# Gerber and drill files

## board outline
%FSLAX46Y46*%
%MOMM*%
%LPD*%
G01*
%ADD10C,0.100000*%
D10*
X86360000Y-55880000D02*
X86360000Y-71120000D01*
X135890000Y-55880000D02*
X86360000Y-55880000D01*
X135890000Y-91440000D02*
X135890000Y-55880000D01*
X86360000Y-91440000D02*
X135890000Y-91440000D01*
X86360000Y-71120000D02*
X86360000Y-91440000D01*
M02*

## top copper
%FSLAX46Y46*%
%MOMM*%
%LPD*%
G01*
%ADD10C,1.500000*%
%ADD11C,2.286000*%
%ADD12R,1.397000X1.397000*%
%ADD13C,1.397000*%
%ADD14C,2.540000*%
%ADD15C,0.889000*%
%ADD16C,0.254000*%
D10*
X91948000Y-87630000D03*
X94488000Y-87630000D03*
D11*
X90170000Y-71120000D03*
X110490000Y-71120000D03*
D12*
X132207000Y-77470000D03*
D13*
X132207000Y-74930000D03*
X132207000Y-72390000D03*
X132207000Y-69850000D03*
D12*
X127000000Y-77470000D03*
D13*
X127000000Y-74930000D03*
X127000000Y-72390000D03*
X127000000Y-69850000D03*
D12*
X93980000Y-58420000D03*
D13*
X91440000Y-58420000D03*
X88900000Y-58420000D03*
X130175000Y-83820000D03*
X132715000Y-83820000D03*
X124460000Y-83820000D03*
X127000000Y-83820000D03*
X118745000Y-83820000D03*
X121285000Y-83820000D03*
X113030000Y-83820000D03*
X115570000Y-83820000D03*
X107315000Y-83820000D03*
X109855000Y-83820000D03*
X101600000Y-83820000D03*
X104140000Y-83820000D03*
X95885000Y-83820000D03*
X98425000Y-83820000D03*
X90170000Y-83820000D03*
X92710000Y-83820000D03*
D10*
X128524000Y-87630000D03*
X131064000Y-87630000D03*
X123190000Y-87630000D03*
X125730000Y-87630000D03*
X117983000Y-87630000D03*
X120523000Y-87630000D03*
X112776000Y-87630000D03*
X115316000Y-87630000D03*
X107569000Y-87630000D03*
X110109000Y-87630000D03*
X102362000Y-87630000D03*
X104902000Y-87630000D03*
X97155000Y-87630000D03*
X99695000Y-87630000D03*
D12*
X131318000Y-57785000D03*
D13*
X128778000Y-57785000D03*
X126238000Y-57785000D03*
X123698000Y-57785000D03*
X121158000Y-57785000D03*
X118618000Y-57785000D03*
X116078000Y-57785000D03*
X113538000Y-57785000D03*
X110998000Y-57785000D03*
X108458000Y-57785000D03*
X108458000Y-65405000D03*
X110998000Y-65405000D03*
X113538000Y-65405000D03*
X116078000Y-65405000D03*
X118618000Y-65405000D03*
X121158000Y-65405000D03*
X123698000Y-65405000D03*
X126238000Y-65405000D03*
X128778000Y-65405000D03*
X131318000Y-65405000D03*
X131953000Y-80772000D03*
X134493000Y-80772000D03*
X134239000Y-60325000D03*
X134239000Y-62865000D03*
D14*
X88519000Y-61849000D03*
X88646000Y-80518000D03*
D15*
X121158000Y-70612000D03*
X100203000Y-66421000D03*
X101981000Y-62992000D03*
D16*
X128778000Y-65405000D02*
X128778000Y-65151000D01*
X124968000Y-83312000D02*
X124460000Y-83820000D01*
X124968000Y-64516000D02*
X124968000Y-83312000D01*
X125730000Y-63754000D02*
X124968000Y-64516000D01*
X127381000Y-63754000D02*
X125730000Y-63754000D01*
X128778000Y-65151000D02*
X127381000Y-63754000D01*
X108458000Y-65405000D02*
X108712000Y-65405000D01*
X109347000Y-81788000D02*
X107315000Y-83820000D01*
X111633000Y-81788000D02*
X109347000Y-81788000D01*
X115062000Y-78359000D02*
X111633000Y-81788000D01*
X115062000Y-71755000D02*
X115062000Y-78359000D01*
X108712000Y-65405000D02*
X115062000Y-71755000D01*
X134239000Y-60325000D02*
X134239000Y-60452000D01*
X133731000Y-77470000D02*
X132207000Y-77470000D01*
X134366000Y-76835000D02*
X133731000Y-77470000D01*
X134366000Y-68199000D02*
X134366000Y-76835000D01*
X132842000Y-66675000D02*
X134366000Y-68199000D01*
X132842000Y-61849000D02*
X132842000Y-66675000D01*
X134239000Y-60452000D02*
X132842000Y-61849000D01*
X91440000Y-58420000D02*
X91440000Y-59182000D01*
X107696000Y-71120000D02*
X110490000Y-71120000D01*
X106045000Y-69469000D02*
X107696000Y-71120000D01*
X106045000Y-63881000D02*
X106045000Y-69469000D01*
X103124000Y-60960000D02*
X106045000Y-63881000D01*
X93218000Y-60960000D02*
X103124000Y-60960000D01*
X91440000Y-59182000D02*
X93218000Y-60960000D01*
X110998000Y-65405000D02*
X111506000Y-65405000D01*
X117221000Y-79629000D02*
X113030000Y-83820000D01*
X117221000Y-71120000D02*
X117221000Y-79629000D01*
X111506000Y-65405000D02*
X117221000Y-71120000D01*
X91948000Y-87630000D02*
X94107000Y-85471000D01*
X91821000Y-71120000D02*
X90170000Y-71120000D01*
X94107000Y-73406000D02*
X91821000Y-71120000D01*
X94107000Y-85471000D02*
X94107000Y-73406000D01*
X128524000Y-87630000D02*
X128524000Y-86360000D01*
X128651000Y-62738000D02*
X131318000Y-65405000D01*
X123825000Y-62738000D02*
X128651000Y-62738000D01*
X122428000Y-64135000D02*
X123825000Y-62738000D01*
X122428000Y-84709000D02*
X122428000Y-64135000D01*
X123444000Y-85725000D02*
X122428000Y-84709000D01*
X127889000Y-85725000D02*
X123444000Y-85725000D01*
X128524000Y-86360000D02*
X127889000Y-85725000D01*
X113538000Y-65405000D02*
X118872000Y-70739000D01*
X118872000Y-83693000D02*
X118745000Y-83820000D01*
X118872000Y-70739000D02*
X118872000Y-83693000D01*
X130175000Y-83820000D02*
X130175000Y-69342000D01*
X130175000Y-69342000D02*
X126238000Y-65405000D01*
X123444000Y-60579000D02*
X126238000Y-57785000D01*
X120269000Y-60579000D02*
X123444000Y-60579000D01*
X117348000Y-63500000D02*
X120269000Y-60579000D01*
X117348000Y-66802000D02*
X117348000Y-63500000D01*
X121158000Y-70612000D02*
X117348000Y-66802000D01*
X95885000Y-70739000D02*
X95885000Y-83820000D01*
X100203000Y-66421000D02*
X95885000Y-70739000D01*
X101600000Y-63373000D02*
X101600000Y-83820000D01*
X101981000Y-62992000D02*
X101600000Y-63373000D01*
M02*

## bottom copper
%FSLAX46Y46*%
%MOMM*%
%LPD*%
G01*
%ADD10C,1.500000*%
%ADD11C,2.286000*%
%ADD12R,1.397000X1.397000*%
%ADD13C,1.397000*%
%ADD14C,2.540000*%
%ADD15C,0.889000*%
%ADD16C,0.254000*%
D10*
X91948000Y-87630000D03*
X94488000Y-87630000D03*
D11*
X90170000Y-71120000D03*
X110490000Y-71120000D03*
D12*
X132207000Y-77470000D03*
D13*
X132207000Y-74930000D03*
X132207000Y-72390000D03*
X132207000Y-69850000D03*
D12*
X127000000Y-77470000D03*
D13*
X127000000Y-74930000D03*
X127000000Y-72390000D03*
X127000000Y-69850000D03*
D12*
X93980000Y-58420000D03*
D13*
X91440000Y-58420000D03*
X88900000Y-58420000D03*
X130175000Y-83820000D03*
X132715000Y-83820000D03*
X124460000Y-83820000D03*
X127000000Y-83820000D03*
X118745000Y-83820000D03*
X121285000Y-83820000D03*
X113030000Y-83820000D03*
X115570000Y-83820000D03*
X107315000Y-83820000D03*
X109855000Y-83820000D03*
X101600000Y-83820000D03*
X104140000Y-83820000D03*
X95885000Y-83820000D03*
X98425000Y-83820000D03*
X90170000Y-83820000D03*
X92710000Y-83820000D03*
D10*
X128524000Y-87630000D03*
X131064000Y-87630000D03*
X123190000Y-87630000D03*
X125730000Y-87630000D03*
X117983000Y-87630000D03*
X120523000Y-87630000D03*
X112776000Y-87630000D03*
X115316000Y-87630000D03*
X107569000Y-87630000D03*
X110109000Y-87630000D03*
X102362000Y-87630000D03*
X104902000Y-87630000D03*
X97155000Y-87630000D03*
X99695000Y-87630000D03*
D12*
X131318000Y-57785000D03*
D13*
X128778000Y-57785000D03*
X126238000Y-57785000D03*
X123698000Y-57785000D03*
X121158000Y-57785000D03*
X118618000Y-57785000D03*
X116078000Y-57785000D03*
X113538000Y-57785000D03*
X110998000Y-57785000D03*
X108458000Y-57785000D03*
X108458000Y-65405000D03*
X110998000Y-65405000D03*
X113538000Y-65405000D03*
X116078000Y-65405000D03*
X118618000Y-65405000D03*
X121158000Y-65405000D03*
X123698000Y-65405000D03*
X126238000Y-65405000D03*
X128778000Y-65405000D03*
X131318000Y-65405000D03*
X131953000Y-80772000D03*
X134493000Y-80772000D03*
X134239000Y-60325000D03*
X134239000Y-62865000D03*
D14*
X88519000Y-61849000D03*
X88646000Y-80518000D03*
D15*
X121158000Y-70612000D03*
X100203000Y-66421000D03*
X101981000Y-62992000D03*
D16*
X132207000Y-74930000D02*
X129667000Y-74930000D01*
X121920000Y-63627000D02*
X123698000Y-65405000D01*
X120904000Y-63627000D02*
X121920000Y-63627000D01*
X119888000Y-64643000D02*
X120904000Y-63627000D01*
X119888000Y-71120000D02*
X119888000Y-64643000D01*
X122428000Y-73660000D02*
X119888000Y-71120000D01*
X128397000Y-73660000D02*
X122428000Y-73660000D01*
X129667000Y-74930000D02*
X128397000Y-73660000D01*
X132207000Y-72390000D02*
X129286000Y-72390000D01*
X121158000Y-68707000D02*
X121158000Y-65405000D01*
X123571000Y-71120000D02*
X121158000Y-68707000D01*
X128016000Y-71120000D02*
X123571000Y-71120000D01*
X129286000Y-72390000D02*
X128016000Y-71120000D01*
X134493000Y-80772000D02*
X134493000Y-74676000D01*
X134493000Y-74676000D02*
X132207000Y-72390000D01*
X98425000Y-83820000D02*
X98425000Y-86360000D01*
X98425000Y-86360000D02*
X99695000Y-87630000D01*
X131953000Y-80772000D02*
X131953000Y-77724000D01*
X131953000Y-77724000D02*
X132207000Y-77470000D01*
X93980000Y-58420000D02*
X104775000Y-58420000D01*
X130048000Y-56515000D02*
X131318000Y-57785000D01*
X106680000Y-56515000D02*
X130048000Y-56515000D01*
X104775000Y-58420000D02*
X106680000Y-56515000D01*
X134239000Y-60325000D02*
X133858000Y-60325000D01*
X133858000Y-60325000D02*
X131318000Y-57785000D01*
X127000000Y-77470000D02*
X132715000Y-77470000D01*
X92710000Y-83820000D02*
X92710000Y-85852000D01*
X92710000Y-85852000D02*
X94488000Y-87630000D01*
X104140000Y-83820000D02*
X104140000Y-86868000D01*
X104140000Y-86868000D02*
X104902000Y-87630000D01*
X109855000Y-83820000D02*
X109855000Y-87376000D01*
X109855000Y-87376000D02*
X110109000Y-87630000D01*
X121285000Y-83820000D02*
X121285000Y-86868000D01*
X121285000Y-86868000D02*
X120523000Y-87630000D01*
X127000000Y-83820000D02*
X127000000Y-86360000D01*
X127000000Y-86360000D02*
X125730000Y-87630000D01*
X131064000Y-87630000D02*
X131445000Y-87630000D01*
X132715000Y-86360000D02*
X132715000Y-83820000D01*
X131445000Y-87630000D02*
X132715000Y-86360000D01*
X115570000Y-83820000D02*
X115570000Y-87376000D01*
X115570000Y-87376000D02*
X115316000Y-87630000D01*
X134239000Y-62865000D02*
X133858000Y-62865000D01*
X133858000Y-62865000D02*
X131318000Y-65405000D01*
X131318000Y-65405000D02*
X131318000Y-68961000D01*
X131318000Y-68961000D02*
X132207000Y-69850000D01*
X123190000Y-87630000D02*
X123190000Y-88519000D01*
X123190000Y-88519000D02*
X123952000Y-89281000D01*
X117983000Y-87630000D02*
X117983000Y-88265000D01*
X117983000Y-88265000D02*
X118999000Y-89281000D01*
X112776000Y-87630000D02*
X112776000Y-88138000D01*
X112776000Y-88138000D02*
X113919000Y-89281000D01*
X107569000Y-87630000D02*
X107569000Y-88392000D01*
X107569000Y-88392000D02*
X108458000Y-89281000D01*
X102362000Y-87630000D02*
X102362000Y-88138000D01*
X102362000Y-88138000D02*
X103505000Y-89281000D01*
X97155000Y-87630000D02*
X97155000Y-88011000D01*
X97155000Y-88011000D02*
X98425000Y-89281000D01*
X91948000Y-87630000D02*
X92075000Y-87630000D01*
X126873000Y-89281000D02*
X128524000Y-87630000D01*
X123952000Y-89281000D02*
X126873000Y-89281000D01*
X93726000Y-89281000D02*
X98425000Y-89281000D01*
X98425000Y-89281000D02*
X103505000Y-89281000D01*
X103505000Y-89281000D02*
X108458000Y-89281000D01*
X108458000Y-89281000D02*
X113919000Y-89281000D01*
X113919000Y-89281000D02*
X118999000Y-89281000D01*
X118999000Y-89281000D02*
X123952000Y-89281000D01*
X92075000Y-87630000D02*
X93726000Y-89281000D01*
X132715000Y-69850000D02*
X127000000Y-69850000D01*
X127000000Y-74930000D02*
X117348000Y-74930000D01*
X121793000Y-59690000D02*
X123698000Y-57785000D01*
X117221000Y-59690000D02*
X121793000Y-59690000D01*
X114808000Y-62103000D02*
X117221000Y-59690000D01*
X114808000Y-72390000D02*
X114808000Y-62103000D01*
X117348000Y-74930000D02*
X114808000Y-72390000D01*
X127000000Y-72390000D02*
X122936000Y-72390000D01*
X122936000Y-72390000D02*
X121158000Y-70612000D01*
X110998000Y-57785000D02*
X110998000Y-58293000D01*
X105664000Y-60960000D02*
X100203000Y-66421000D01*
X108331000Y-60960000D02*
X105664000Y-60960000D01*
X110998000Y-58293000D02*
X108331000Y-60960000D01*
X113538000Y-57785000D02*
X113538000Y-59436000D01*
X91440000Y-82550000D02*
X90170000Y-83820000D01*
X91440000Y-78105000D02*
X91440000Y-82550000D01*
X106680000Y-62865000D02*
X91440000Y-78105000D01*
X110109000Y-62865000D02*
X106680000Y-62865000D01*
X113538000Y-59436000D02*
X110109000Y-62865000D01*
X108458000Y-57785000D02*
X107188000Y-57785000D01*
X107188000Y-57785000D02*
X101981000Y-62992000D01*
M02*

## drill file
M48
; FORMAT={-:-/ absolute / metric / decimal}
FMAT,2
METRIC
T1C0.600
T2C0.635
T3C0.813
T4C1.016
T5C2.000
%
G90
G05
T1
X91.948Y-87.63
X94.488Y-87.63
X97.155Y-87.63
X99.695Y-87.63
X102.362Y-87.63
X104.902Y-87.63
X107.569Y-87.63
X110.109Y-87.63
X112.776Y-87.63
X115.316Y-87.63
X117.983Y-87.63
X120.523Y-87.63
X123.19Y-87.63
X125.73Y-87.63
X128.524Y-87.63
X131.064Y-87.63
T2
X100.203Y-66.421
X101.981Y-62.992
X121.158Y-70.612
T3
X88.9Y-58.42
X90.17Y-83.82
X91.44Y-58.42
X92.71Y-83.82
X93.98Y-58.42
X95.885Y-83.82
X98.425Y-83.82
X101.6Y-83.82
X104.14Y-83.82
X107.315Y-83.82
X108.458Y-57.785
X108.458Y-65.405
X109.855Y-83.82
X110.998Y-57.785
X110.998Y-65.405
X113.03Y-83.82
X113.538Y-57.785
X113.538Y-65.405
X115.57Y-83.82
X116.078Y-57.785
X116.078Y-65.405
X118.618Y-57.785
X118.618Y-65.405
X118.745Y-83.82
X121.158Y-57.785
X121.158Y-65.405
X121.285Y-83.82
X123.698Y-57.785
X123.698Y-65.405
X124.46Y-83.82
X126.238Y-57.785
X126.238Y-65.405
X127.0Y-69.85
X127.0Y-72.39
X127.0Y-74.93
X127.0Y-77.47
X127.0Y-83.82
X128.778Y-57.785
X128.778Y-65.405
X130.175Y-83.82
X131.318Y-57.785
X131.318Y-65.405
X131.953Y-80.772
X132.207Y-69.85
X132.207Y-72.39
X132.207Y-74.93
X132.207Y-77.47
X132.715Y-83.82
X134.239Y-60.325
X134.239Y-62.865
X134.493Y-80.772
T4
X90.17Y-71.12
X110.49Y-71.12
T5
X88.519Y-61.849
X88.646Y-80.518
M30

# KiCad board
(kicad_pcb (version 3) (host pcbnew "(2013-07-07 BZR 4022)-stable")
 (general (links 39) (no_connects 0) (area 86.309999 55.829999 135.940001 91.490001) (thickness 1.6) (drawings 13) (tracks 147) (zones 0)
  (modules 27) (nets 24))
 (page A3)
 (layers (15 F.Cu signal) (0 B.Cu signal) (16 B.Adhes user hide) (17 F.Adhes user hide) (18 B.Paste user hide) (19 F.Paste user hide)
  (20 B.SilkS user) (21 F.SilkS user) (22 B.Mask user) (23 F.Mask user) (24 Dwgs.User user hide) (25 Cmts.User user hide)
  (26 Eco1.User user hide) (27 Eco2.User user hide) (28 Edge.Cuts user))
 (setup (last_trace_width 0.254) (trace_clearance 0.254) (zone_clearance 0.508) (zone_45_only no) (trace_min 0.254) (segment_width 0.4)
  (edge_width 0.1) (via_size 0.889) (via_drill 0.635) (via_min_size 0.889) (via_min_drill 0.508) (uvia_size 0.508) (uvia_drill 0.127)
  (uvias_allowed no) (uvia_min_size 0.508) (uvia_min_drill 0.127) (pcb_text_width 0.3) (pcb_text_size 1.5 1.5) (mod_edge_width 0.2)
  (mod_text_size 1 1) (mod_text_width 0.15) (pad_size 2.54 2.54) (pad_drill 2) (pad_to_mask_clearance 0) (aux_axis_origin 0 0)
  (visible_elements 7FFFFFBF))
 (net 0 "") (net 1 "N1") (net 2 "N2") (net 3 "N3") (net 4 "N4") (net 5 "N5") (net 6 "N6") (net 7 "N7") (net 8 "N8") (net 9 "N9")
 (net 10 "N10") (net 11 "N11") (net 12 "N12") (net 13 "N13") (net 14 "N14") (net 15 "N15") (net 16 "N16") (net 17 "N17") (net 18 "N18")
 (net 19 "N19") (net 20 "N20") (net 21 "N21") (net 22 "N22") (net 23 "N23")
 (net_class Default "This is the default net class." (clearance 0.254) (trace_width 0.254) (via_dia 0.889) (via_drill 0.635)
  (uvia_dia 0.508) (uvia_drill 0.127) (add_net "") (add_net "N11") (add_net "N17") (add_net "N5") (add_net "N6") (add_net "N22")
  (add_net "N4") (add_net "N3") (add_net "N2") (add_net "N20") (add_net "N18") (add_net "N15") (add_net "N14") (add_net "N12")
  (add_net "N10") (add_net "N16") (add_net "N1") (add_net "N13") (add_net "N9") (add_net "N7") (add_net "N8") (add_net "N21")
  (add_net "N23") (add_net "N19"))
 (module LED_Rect (layer F.Cu) (at 91.948 87.63)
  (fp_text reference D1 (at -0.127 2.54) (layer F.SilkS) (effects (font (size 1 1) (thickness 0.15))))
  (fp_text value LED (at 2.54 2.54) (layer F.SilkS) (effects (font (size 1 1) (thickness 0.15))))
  (pad 1 thru_hole circle (at 0 0) (size 1.5 1.5) (drill 0.6) (layers *.Cu *.Mask F.SilkS) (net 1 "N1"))
  (pad 2 thru_hole circle (at 2.54 0) (size 1.5 1.5) (drill 0.6) (layers *.Cu *.Mask F.SilkS) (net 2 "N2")))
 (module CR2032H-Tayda (layer F.Cu) (at 97.79 71.12)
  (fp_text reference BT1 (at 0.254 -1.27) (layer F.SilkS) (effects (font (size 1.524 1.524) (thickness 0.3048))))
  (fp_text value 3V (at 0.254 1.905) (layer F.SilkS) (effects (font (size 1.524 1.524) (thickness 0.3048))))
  (pad 2 thru_hole circle (at -7.62 0) (size 2.286 2.286) (drill 1.016) (layers *.Cu *.Mask F.SilkS) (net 1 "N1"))
  (pad 1 thru_hole circle (at 12.7 0) (size 2.286 2.286) (drill 1.016) (layers *.Cu *.Mask F.SilkS) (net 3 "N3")))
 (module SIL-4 (layer F.Cu) (at 132.207 73.66 90)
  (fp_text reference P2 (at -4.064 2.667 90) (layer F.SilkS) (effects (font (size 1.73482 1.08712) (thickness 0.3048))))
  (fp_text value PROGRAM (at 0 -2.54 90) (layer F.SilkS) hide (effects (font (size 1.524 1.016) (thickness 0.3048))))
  (pad 1 thru_hole rect (at -3.81 0 90) (size 1.397 1.397) (drill 0.8128) (layers *.Cu *.Mask F.SilkS) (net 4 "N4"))
  (pad 2 thru_hole circle (at -1.27 0 90) (size 1.397 1.397) (drill 0.8128) (layers *.Cu *.Mask F.SilkS) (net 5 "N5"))
  (pad 3 thru_hole circle (at 1.27 0 90) (size 1.397 1.397) (drill 0.8128) (layers *.Cu *.Mask F.SilkS) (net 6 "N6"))
  (pad 4 thru_hole circle (at 3.81 0 90) (size 1.397 1.397) (drill 0.8128) (layers *.Cu *.Mask F.SilkS) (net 1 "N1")))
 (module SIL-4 (layer F.Cu) (at 127 73.66 90)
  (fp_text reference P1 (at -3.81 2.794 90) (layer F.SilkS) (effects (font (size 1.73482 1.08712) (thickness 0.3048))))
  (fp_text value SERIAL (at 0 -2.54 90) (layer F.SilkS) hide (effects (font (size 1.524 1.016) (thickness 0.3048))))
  (pad 1 thru_hole rect (at -3.81 0 90) (size 1.397 1.397) (drill 0.8128) (layers *.Cu *.Mask F.SilkS) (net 4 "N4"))
  (pad 2 thru_hole circle (at -1.27 0 90) (size 1.397 1.397) (drill 0.8128) (layers *.Cu *.Mask F.SilkS) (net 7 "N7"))
  (pad 3 thru_hole circle (at 1.27 0 90) (size 1.397 1.397) (drill 0.8128) (layers *.Cu *.Mask F.SilkS) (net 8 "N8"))
  (pad 4 thru_hole circle (at 3.81 0 90) (size 1.397 1.397) (drill 0.8128) (layers *.Cu *.Mask F.SilkS) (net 1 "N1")))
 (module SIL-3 (layer F.Cu) (at 91.44 58.42 180)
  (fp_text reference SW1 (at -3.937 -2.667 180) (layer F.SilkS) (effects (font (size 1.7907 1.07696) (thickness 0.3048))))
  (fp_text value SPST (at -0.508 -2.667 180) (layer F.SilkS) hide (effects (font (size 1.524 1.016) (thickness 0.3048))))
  (pad 1 thru_hole rect (at -2.54 0 180) (size 1.397 1.397) (drill 0.8128) (layers *.Cu *.Mask F.SilkS) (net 4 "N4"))
  (pad 2 thru_hole circle (at 0 0 180) (size 1.397 1.397) (drill 0.8128) (layers *.Cu *.Mask F.SilkS) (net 3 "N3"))
  (pad 3 thru_hole circle (at 2.54 0 180) (size 1.397 1.397) (drill 0.8128) (layers *.Cu *.Mask F.SilkS)))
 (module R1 (layer F.Cu) (at 131.445 83.82) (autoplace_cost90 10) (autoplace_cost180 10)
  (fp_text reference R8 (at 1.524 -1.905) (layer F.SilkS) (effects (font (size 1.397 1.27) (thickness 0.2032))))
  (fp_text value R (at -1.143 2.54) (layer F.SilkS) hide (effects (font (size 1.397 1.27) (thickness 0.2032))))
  (pad 1 thru_hole circle (at -1.27 0) (size 1.397 1.397) (drill 0.8128) (layers *.Cu *.Mask F.SilkS) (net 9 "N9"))
  (pad 2 thru_hole circle (at 1.27 0) (size 1.397 1.397) (drill 0.8128) (layers *.Cu *.Mask F.SilkS) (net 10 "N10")))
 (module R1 (layer F.Cu) (at 125.73 83.82) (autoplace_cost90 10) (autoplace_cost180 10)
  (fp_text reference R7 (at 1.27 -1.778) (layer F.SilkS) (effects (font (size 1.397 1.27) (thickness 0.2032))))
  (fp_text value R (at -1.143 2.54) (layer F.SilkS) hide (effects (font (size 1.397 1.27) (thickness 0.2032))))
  (pad 1 thru_hole circle (at -1.27 0) (size 1.397 1.397) (drill 0.8128) (layers *.Cu *.Mask F.SilkS) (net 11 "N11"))
  (pad 2 thru_hole circle (at 1.27 0) (size 1.397 1.397) (drill 0.8128) (layers *.Cu *.Mask F.SilkS) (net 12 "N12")))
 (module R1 (layer F.Cu) (at 120.015 83.82) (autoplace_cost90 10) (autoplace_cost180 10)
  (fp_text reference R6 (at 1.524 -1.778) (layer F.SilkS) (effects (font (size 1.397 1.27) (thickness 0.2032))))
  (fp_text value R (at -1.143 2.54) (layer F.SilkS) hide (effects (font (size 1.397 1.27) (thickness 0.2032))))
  (pad 1 thru_hole circle (at -1.27 0) (size 1.397 1.397) (drill 0.8128) (layers *.Cu *.Mask F.SilkS) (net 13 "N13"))
  (pad 2 thru_hole circle (at 1.27 0) (size 1.397 1.397) (drill 0.8128) (layers *.Cu *.Mask F.SilkS) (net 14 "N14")))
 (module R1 (layer F.Cu) (at 114.3 83.82) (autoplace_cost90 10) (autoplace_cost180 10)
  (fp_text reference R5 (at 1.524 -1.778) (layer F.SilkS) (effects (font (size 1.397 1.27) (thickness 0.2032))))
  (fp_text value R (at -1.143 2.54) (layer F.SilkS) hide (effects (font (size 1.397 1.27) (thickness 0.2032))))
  (pad 1 thru_hole circle (at -1.27 0) (size 1.397 1.397) (drill 0.8128) (layers *.Cu *.Mask F.SilkS) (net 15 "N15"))
  (pad 2 thru_hole circle (at 1.27 0) (size 1.397 1.397) (drill 0.8128) (layers *.Cu *.Mask F.SilkS) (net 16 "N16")))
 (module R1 (layer F.Cu) (at 108.585 83.82) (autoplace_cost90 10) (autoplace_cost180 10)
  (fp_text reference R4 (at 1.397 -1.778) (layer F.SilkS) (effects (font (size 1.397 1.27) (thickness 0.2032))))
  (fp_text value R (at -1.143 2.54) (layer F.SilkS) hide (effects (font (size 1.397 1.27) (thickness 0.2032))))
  (pad 1 thru_hole circle (at -1.27 0) (size 1.397 1.397) (drill 0.8128) (layers *.Cu *.Mask F.SilkS) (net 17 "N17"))
  (pad 2 thru_hole circle (at 1.27 0) (size 1.397 1.397) (drill 0.8128) (layers *.Cu *.Mask F.SilkS) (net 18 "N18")))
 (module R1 (layer F.Cu) (at 102.87 83.82) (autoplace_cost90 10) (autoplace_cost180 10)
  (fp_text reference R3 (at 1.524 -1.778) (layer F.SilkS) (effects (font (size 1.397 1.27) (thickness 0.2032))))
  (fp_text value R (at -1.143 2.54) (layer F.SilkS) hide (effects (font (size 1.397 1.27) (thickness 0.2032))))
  (pad 1 thru_hole circle (at -1.27 0) (size 1.397 1.397) (drill 0.8128) (layers *.Cu *.Mask F.SilkS) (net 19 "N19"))
  (pad 2 thru_hole circle (at 1.27 0) (size 1.397 1.397) (drill 0.8128) (layers *.Cu *.Mask F.SilkS) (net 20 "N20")))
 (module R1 (layer F.Cu) (at 97.155 83.82) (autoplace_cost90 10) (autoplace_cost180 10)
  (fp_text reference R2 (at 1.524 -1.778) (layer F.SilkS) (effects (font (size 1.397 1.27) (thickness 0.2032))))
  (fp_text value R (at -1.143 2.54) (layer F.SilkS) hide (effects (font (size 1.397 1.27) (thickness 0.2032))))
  (pad 1 thru_hole circle (at -1.27 0) (size 1.397 1.397) (drill 0.8128) (layers *.Cu *.Mask F.SilkS) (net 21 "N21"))
  (pad 2 thru_hole circle (at 1.27 0) (size 1.397 1.397) (drill 0.8128) (layers *.Cu *.Mask F.SilkS) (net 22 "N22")))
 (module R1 (layer F.Cu) (at 91.44 83.82) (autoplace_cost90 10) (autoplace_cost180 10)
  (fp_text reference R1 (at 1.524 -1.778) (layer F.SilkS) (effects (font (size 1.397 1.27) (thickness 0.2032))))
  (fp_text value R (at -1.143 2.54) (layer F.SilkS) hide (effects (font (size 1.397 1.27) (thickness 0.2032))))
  (pad 1 thru_hole circle (at -1.27 0) (size 1.397 1.397) (drill 0.8128) (layers *.Cu *.Mask F.SilkS) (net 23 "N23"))
  (pad 2 thru_hole circle (at 1.27 0) (size 1.397 1.397) (drill 0.8128) (layers *.Cu *.Mask F.SilkS) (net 2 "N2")))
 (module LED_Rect (layer F.Cu) (at 128.524 87.63)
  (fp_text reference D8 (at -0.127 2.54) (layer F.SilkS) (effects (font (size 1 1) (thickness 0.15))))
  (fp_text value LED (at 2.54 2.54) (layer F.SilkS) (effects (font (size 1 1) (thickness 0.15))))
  (pad 1 thru_hole circle (at 0 0) (size 1.5 1.5) (drill 0.6) (layers *.Cu *.Mask F.SilkS) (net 1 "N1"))
  (pad 2 thru_hole circle (at 2.54 0) (size 1.5 1.5) (drill 0.6) (layers *.Cu *.Mask F.SilkS) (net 10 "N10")))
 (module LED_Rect (layer F.Cu) (at 123.19 87.63)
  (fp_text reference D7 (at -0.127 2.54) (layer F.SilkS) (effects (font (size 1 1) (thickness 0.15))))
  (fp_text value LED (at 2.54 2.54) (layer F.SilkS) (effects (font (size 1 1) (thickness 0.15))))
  (pad 1 thru_hole circle (at 0 0) (size 1.5 1.5) (drill 0.6) (layers *.Cu *.Mask F.SilkS) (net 1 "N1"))
  (pad 2 thru_hole circle (at 2.54 0) (size 1.5 1.5) (drill 0.6) (layers *.Cu *.Mask F.SilkS) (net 12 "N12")))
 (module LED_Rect (layer F.Cu) (at 117.983 87.63)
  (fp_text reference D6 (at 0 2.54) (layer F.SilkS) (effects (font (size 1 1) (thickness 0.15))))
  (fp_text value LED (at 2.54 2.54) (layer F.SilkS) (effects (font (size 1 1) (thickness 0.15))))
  (pad 1 thru_hole circle (at 0 0) (size 1.5 1.5) (drill 0.6) (layers *.Cu *.Mask F.SilkS) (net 1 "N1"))
  (pad 2 thru_hole circle (at 2.54 0) (size 1.5 1.5) (drill 0.6) (layers *.Cu *.Mask F.SilkS) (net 14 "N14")))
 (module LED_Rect (layer F.Cu) (at 112.776 87.63)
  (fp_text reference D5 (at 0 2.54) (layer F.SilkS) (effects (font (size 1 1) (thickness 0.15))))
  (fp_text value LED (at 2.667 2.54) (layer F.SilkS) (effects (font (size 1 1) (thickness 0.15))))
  (pad 1 thru_hole circle (at 0 0) (size 1.5 1.5) (drill 0.6) (layers *.Cu *.Mask F.SilkS) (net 1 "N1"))
  (pad 2 thru_hole circle (at 2.54 0) (size 1.5 1.5) (drill 0.6) (layers *.Cu *.Mask F.SilkS) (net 16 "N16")))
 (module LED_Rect (layer F.Cu) (at 107.569 87.63)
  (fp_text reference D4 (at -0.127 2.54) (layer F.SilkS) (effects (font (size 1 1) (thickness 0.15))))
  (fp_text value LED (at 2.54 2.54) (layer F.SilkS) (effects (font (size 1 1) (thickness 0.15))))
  (pad 1 thru_hole circle (at 0 0) (size 1.5 1.5) (drill 0.6) (layers *.Cu *.Mask F.SilkS) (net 1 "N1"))
  (pad 2 thru_hole circle (at 2.54 0) (size 1.5 1.5) (drill 0.6) (layers *.Cu *.Mask F.SilkS) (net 18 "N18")))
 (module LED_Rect (layer F.Cu) (at 102.362 87.63)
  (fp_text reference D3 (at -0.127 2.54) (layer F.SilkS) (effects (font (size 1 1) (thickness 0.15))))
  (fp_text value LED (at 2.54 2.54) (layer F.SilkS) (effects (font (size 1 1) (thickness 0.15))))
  (pad 1 thru_hole circle (at 0 0) (size 1.5 1.5) (drill 0.6) (layers *.Cu *.Mask F.SilkS) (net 1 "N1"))
  (pad 2 thru_hole circle (at 2.54 0) (size 1.5 1.5) (drill 0.6) (layers *.Cu *.Mask F.SilkS) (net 20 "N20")))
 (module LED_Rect (layer F.Cu) (at 97.155 87.63)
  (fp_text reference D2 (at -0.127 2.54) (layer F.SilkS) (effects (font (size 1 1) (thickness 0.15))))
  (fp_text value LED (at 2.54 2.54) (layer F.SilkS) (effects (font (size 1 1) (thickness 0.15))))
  (pad 1 thru_hole circle (at 0 0) (size 1.5 1.5) (drill 0.6) (layers *.Cu *.Mask F.SilkS) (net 1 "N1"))
  (pad 2 thru_hole circle (at 2.54 0) (size 1.5 1.5) (drill 0.6) (layers *.Cu *.Mask F.SilkS) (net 22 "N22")))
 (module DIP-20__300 (layer F.Cu) (at 119.888 61.595 180)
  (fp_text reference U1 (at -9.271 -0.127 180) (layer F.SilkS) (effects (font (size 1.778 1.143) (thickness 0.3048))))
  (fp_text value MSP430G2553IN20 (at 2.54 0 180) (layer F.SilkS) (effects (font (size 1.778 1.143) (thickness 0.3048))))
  (pad 1 thru_hole rect (at -11.43 3.81 180) (size 1.397 1.397) (drill 0.8128) (layers *.Cu *.Mask F.SilkS) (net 4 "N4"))
  (pad 2 thru_hole circle (at -8.89 3.81 180) (size 1.397 1.397) (drill 0.8128) (layers *.Cu *.Mask F.SilkS))
  (pad 3 thru_hole circle (at -6.35 3.81 180) (size 1.397 1.397) (drill 0.8128) (layers *.Cu *.Mask F.SilkS) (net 8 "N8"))
  (pad 4 thru_hole circle (at -3.81 3.81 180) (size 1.397 1.397) (drill 0.8128) (layers *.Cu *.Mask F.SilkS) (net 7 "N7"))
  (pad 5 thru_hole circle (at -1.27 3.81 180) (size 1.397 1.397) (drill 0.8128) (layers *.Cu *.Mask F.SilkS))
  (pad 6 thru_hole circle (at 1.27 3.81 180) (size 1.397 1.397) (drill 0.8128) (layers *.Cu *.Mask F.SilkS))
  (pad 7 thru_hole circle (at 3.81 3.81 180) (size 1.397 1.397) (drill 0.8128) (layers *.Cu *.Mask F.SilkS))
  (pad 8 thru_hole circle (at 6.35 3.81 180) (size 1.397 1.397) (drill 0.8128) (layers *.Cu *.Mask F.SilkS) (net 23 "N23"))
  (pad 9 thru_hole circle (at 8.89 3.81 180) (size 1.397 1.397) (drill 0.8128) (layers *.Cu *.Mask F.SilkS) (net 21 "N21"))
  (pad 10 thru_hole circle (at 11.43 3.81 180) (size 1.397 1.397) (drill 0.8128) (layers *.Cu *.Mask F.SilkS) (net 19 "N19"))
  (pad 11 thru_hole circle (at 11.43 -3.81 180) (size 1.397 1.397) (drill 0.8128) (layers *.Cu *.Mask F.SilkS) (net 17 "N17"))
  (pad 12 thru_hole circle (at 8.89 -3.81 180) (size 1.397 1.397) (drill 0.8128) (layers *.Cu *.Mask F.SilkS) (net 15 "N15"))
  (pad 13 thru_hole circle (at 6.35 -3.81 180) (size 1.397 1.397) (drill 0.8128) (layers *.Cu *.Mask F.SilkS) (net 13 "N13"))
  (pad 14 thru_hole circle (at 3.81 -3.81 180) (size 1.397 1.397) (drill 0.8128) (layers *.Cu *.Mask F.SilkS))
  (pad 15 thru_hole circle (at 1.27 -3.81 180) (size 1.397 1.397) (drill 0.8128) (layers *.Cu *.Mask F.SilkS))
  (pad 16 thru_hole circle (at -1.27 -3.81 180) (size 1.397 1.397) (drill 0.8128) (layers *.Cu *.Mask F.SilkS) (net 6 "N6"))
  (pad 17 thru_hole circle (at -3.81 -3.81 180) (size 1.397 1.397) (drill 0.8128) (layers *.Cu *.Mask F.SilkS) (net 5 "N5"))
  (pad 18 thru_hole circle (at -6.35 -3.81 180) (size 1.397 1.397) (drill 0.8128) (layers *.Cu *.Mask F.SilkS) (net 9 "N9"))
  (pad 19 thru_hole circle (at -8.89 -3.81 180) (size 1.397 1.397) (drill 0.8128) (layers *.Cu *.Mask F.SilkS) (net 11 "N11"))
  (pad 20 thru_hole circle (at -11.43 -3.81 180) (size 1.397 1.397) (drill 0.8128) (layers *.Cu *.Mask F.SilkS) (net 1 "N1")))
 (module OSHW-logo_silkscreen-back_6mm (layer F.Cu) (at 97.409 65.405)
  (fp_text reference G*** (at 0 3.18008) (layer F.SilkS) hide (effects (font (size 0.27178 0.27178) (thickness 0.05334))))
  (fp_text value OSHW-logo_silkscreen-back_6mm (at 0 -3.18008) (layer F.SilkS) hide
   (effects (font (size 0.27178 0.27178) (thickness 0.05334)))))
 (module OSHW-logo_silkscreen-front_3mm (layer F.Cu) (at 119.38 68.072)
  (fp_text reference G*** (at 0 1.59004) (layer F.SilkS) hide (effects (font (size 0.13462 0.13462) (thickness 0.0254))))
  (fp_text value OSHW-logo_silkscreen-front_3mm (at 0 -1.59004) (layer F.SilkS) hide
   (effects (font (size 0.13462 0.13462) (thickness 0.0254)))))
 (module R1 (layer F.Cu) (at 133.223 80.772) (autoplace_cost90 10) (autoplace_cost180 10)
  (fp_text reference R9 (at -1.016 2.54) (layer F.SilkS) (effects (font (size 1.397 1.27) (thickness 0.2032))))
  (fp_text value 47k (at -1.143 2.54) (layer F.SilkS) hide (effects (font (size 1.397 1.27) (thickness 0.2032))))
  (pad 1 thru_hole circle (at -1.27 0) (size 1.397 1.397) (drill 0.8128) (layers *.Cu *.Mask F.SilkS) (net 4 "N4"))
  (pad 2 thru_hole circle (at 1.27 0) (size 1.397 1.397) (drill 0.8128) (layers *.Cu *.Mask F.SilkS) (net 6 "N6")))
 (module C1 (layer F.Cu) (at 134.239 61.595 270)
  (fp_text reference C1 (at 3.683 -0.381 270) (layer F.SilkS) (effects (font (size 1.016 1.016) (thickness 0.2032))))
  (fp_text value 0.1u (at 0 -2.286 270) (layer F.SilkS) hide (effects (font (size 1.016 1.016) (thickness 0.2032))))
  (pad 1 thru_hole circle (at -1.27 0 270) (size 1.397 1.397) (drill 0.8128) (layers *.Cu *.Mask F.SilkS) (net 4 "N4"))
  (pad 2 thru_hole circle (at 1.27 0 270) (size 1.397 1.397) (drill 0.8128) (layers *.Cu *.Mask F.SilkS) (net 1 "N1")))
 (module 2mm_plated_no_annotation (layer F.Cu) (at 88.519 61.849)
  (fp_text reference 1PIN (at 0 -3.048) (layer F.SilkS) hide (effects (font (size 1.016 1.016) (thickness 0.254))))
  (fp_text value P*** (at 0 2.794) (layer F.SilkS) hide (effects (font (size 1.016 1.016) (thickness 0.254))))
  (pad "" thru_hole circle (at 0 0) (size 2.54 2.54) (drill 2) (layers *.Cu *.Mask F.SilkS)))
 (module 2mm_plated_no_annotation (layer F.Cu) (at 88.646 80.518)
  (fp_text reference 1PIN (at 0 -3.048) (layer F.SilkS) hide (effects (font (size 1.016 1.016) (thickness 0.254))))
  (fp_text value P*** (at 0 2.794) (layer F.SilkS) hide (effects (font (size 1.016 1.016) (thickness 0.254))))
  (pad "" thru_hole circle (at 0 0) (size 2.54 2.54) (drill 2) (layers *.Cu *.Mask F.SilkS)))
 (gr_line (start 86.36 55.88) (end 86.36 71.12) (angle 90) (layer Edge.Cuts) (width 0.1))
 (gr_line (start 135.89 55.88) (end 86.36 55.88) (angle 90) (layer Edge.Cuts) (width 0.1))
 (gr_line (start 135.89 91.44) (end 135.89 55.88) (angle 90) (layer Edge.Cuts) (width 0.1))
 (gr_line (start 86.36 91.44) (end 135.89 91.44) (angle 90) (layer Edge.Cuts) (width 0.1))
 (gr_line (start 86.36 71.12) (end 86.36 91.44) (angle 90) (layer Edge.Cuts) (width 0.1))
 (segment (start 128.778 65.405) (end 128.778 65.151) (width 0.254) (layer F.Cu) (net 11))
 (segment (start 124.968 83.312) (end 124.46 83.82) (width 0.254) (layer F.Cu) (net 11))
 (segment (start 124.968 64.516) (end 124.968 83.312) (width 0.254) (layer F.Cu) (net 11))
 (segment (start 125.73 63.754) (end 124.968 64.516) (width 0.254) (layer F.Cu) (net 11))
 (segment (start 127.381 63.754) (end 125.73 63.754) (width 0.254) (layer F.Cu) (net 11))
 (segment (start 128.778 65.151) (end 127.381 63.754) (width 0.254) (layer F.Cu) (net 11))
 (segment (start 108.458 65.405) (end 108.712 65.405) (width 0.254) (layer F.Cu) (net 17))
 (segment (start 109.347 81.788) (end 107.315 83.82) (width 0.254) (layer F.Cu) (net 17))
 (segment (start 111.633 81.788) (end 109.347 81.788) (width 0.254) (layer F.Cu) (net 17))
 (segment (start 115.062 78.359) (end 111.633 81.788) (width 0.254) (layer F.Cu) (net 17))
 (segment (start 115.062 71.755) (end 115.062 78.359) (width 0.254) (layer F.Cu) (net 17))
 (segment (start 108.712 65.405) (end 115.062 71.755) (width 0.254) (layer F.Cu) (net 17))
 (segment (start 132.207 74.93) (end 129.667 74.93) (width 0.254) (layer B.Cu) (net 5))
 (segment (start 121.92 63.627) (end 123.698 65.405) (width 0.254) (layer B.Cu) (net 5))
 (segment (start 120.904 63.627) (end 121.92 63.627) (width 0.254) (layer B.Cu) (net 5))
 (segment (start 119.888 64.643) (end 120.904 63.627) (width 0.254) (layer B.Cu) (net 5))
 (segment (start 119.888 71.12) (end 119.888 64.643) (width 0.254) (layer B.Cu) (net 5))
 (segment (start 122.428 73.66) (end 119.888 71.12) (width 0.254) (layer B.Cu) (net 5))
 (segment (start 128.397 73.66) (end 122.428 73.66) (width 0.254) (layer B.Cu) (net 5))
 (segment (start 129.667 74.93) (end 128.397 73.66) (width 0.254) (layer B.Cu) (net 5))
 (segment (start 132.207 72.39) (end 129.286 72.39) (width 0.254) (layer B.Cu) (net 6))
 (segment (start 121.158 68.707) (end 121.158 65.405) (width 0.254) (layer B.Cu) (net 6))
 (segment (start 123.571 71.12) (end 121.158 68.707) (width 0.254) (layer B.Cu) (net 6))
 (segment (start 128.016 71.12) (end 123.571 71.12) (width 0.254) (layer B.Cu) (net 6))
 (segment (start 129.286 72.39) (end 128.016 71.12) (width 0.254) (layer B.Cu) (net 6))
 (segment (start 134.493 80.772) (end 134.493 74.676) (width 0.254) (layer B.Cu) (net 6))
 (segment (start 134.493 74.676) (end 132.207 72.39) (width 0.254) (layer B.Cu) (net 6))
 (segment (start 98.425 83.82) (end 98.425 86.36) (width 0.254) (layer B.Cu) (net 22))
 (segment (start 98.425 86.36) (end 99.695 87.63) (width 0.254) (layer B.Cu) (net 22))
 (segment (start 131.953 80.772) (end 131.953 77.724) (width 0.254) (layer B.Cu) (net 4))
 (segment (start 131.953 77.724) (end 132.207 77.47) (width 0.254) (layer B.Cu) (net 4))
 (segment (start 134.239 60.325) (end 134.239 60.452) (width 0.254) (layer F.Cu) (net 4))
 (segment (start 133.731 77.47) (end 132.207 77.47) (width 0.254) (layer F.Cu) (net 4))
 (segment (start 134.366 76.835) (end 133.731 77.47) (width 0.254) (layer F.Cu) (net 4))
 (segment (start 134.366 68.199) (end 134.366 76.835) (width 0.254) (layer F.Cu) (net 4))
 (segment (start 132.842 66.675) (end 134.366 68.199) (width 0.254) (layer F.Cu) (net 4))
 (segment (start 132.842 61.849) (end 132.842 66.675) (width 0.254) (layer F.Cu) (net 4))
 (segment (start 134.239 60.452) (end 132.842 61.849) (width 0.254) (layer F.Cu) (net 4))
 (segment (start 93.98 58.42) (end 104.775 58.42) (width 0.254) (layer B.Cu) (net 4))
 (segment (start 130.048 56.515) (end 131.318 57.785) (width 0.254) (layer B.Cu) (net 4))
 (segment (start 106.68 56.515) (end 130.048 56.515) (width 0.254) (layer B.Cu) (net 4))
 (segment (start 104.775 58.42) (end 106.68 56.515) (width 0.254) (layer B.Cu) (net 4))
 (segment (start 134.239 60.325) (end 133.858 60.325) (width 0.254) (layer B.Cu) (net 4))
 (segment (start 133.858 60.325) (end 131.318 57.785) (width 0.254) (layer B.Cu) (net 4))
 (segment (start 127 77.47) (end 132.715 77.47) (width 0.254) (layer B.Cu) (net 4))
 (segment (start 91.44 58.42) (end 91.44 59.182) (width 0.254) (layer F.Cu) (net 3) (status 400000))
 (segment (start 107.696 71.12) (end 110.49 71.12) (width 0.254) (layer F.Cu) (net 3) (status 800000))
 (segment (start 106.045 69.469) (end 107.696 71.12) (width 0.254) (layer F.Cu) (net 3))
 (segment (start 106.045 63.881) (end 106.045 69.469) (width 0.254) (layer F.Cu) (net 3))
 (segment (start 103.124 60.96) (end 106.045 63.881) (width 0.254) (layer F.Cu) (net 3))
 (segment (start 93.218 60.96) (end 103.124 60.96) (width 0.254) (layer F.Cu) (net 3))
 (segment (start 91.44 59.182) (end 93.218 60.96) (width 0.254) (layer F.Cu) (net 3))
 (segment (start 92.71 83.82) (end 92.71 85.852) (width 0.254) (layer B.Cu) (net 2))
 (segment (start 92.71 85.852) (end 94.488 87.63) (width 0.254) (layer B.Cu) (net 2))
 (segment (start 104.14 83.82) (end 104.14 86.868) (width 0.254) (layer B.Cu) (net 20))
 (segment (start 104.14 86.868) (end 104.902 87.63) (width 0.254) (layer B.Cu) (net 20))
 (segment (start 109.855 83.82) (end 109.855 87.376) (width 0.254) (layer B.Cu) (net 18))
 (segment (start 109.855 87.376) (end 110.109 87.63) (width 0.254) (layer B.Cu) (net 18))
 (segment (start 110.998 65.405) (end 111.506 65.405) (width 0.254) (layer F.Cu) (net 15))
 (segment (start 117.221 79.629) (end 113.03 83.82) (width 0.254) (layer F.Cu) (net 15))
 (segment (start 117.221 71.12) (end 117.221 79.629) (width 0.254) (layer F.Cu) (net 15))
 (segment (start 111.506 65.405) (end 117.221 71.12) (width 0.254) (layer F.Cu) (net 15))
 (segment (start 121.285 83.82) (end 121.285 86.868) (width 0.254) (layer B.Cu) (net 14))
 (segment (start 121.285 86.868) (end 120.523 87.63) (width 0.254) (layer B.Cu) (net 14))
 (segment (start 127 83.82) (end 127 86.36) (width 0.254) (layer B.Cu) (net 12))
 (segment (start 127 86.36) (end 125.73 87.63) (width 0.254) (layer B.Cu) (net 12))
 (segment (start 131.064 87.63) (end 131.445 87.63) (width 0.254) (layer B.Cu) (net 10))
 (segment (start 132.715 86.36) (end 132.715 83.82) (width 0.254) (layer B.Cu) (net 10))
 (segment (start 131.445 87.63) (end 132.715 86.36) (width 0.254) (layer B.Cu) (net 10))
 (segment (start 115.57 83.82) (end 115.57 87.376) (width 0.254) (layer B.Cu) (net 16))
 (segment (start 115.57 87.376) (end 115.316 87.63) (width 0.254) (layer B.Cu) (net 16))
 (segment (start 91.948 87.63) (end 94.107 85.471) (width 0.254) (layer F.Cu) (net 1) (status 400000))
 (segment (start 91.821 71.12) (end 90.17 71.12) (width 0.254) (layer F.Cu) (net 1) (status 800000))
 (segment (start 94.107 73.406) (end 91.821 71.12) (width 0.254) (layer F.Cu) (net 1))
 (segment (start 94.107 85.471) (end 94.107 73.406) (width 0.254) (layer F.Cu) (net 1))
 (segment (start 128.524 87.63) (end 128.524 86.36) (width 0.254) (layer F.Cu) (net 1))
 (segment (start 128.651 62.738) (end 131.318 65.405) (width 0.254) (layer F.Cu) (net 1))
 (segment (start 123.825 62.738) (end 128.651 62.738) (width 0.254) (layer F.Cu) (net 1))
 (segment (start 122.428 64.135) (end 123.825 62.738) (width 0.254) (layer F.Cu) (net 1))
 (segment (start 122.428 84.709) (end 122.428 64.135) (width 0.254) (layer F.Cu) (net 1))
 (segment (start 123.444 85.725) (end 122.428 84.709) (width 0.254) (layer F.Cu) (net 1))
 (segment (start 127.889 85.725) (end 123.444 85.725) (width 0.254) (layer F.Cu) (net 1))
 (segment (start 128.524 86.36) (end 127.889 85.725) (width 0.254) (layer F.Cu) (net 1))
 (segment (start 134.239 62.865) (end 133.858 62.865) (width 0.254) (layer B.Cu) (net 1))
 (segment (start 133.858 62.865) (end 131.318 65.405) (width 0.254) (layer B.Cu) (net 1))
 (segment (start 131.318 65.405) (end 131.318 68.961) (width 0.254) (layer B.Cu) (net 1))
 (segment (start 131.318 68.961) (end 132.207 69.85) (width 0.254) (layer B.Cu) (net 1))
 (segment (start 123.19 87.63) (end 123.19 88.519) (width 0.254) (layer B.Cu) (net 1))
 (segment (start 123.19 88.519) (end 123.952 89.281) (width 0.254) (layer B.Cu) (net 1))
 (segment (start 117.983 87.63) (end 117.983 88.265) (width 0.254) (layer B.Cu) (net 1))
 (segment (start 117.983 88.265) (end 118.999 89.281) (width 0.254) (layer B.Cu) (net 1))
 (segment (start 112.776 87.63) (end 112.776 88.138) (width 0.254) (layer B.Cu) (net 1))
 (segment (start 112.776 88.138) (end 113.919 89.281) (width 0.254) (layer B.Cu) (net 1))
 (segment (start 107.569 87.63) (end 107.569 88.392) (width 0.254) (layer B.Cu) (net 1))
 (segment (start 107.569 88.392) (end 108.458 89.281) (width 0.254) (layer B.Cu) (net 1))
 (segment (start 102.362 87.63) (end 102.362 88.138) (width 0.254) (layer B.Cu) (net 1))
 (segment (start 102.362 88.138) (end 103.505 89.281) (width 0.254) (layer B.Cu) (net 1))
 (segment (start 97.155 87.63) (end 97.155 88.011) (width 0.254) (layer B.Cu) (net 1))
 (segment (start 97.155 88.011) (end 98.425 89.281) (width 0.254) (layer B.Cu) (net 1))
 (segment (start 91.948 87.63) (end 92.075 87.63) (width 0.254) (layer B.Cu) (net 1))
 (segment (start 126.873 89.281) (end 128.524 87.63) (width 0.254) (layer B.Cu) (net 1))
 (segment (start 123.952 89.281) (end 126.873 89.281) (width 0.254) (layer B.Cu) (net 1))
 (segment (start 93.726 89.281) (end 98.425 89.281) (width 0.254) (layer B.Cu) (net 1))
 (segment (start 98.425 89.281) (end 103.505 89.281) (width 0.254) (layer B.Cu) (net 1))
 (segment (start 103.505 89.281) (end 108.458 89.281) (width 0.254) (layer B.Cu) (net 1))
 (segment (start 108.458 89.281) (end 113.919 89.281) (width 0.254) (layer B.Cu) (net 1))
 (segment (start 113.919 89.281) (end 118.999 89.281) (width 0.254) (layer B.Cu) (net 1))
 (segment (start 118.999 89.281) (end 123.952 89.281) (width 0.254) (layer B.Cu) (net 1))
 (segment (start 92.075 87.63) (end 93.726 89.281) (width 0.254) (layer B.Cu) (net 1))
 (segment (start 132.715 69.85) (end 127 69.85) (width 0.254) (layer B.Cu) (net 1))
 (segment (start 113.538 65.405) (end 118.872 70.739) (width 0.254) (layer F.Cu) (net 13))
 (segment (start 118.872 83.693) (end 118.745 83.82) (width 0.254) (layer F.Cu) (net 13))
 (segment (start 118.872 70.739) (end 118.872 83.693) (width 0.254) (layer F.Cu) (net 13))
 (segment (start 130.175 83.82) (end 130.175 69.342) (width 0.254) (layer F.Cu) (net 9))
 (segment (start 130.175 69.342) (end 126.238 65.405) (width 0.254) (layer F.Cu) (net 9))
 (segment (start 127 74.93) (end 117.348 74.93) (width 0.254) (layer B.Cu) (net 7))
 (segment (start 121.793 59.69) (end 123.698 57.785) (width 0.254) (layer B.Cu) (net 7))
 (segment (start 117.221 59.69) (end 121.793 59.69) (width 0.254) (layer B.Cu) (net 7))
 (segment (start 114.808 62.103) (end 117.221 59.69) (width 0.254) (layer B.Cu) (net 7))
 (segment (start 114.808 72.39) (end 114.808 62.103) (width 0.254) (layer B.Cu) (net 7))
 (segment (start 117.348 74.93) (end 114.808 72.39) (width 0.254) (layer B.Cu) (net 7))
 (segment (start 127 72.39) (end 122.936 72.39) (width 0.254) (layer B.Cu) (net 8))
 (segment (start 123.444 60.579) (end 126.238 57.785) (width 0.254) (layer F.Cu) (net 8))
 (segment (start 120.269 60.579) (end 123.444 60.579) (width 0.254) (layer F.Cu) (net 8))
 (segment (start 117.348 63.5) (end 120.269 60.579) (width 0.254) (layer F.Cu) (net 8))
 (segment (start 117.348 66.802) (end 117.348 63.5) (width 0.254) (layer F.Cu) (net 8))
 (segment (start 121.158 70.612) (end 117.348 66.802) (width 0.254) (layer F.Cu) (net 8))
 (via (at 121.158 70.612) (size 0.889) (layers F.Cu B.Cu) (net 8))
 (segment (start 122.936 72.39) (end 121.158 70.612) (width 0.254) (layer B.Cu) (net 8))
 (segment (start 110.998 57.785) (end 110.998 58.293) (width 0.254) (layer B.Cu) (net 21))
 (segment (start 95.885 70.739) (end 95.885 83.82) (width 0.254) (layer F.Cu) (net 21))
 (segment (start 100.203 66.421) (end 95.885 70.739) (width 0.254) (layer F.Cu) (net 21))
 (via (at 100.203 66.421) (size 0.889) (layers F.Cu B.Cu) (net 21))
 (segment (start 105.664 60.96) (end 100.203 66.421) (width 0.254) (layer B.Cu) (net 21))
 (segment (start 108.331 60.96) (end 105.664 60.96) (width 0.254) (layer B.Cu) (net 21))
 (segment (start 110.998 58.293) (end 108.331 60.96) (width 0.254) (layer B.Cu) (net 21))
 (segment (start 113.538 57.785) (end 113.538 59.436) (width 0.254) (layer B.Cu) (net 23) (status 400000))
 (segment (start 91.44 82.55) (end 90.17 83.82) (width 0.254) (layer B.Cu) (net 23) (status 800000))
 (segment (start 91.44 78.105) (end 91.44 82.55) (width 0.254) (layer B.Cu) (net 23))
 (segment (start 106.68 62.865) (end 91.44 78.105) (width 0.254) (layer B.Cu) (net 23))
 (segment (start 110.109 62.865) (end 106.68 62.865) (width 0.254) (layer B.Cu) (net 23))
 (segment (start 113.538 59.436) (end 110.109 62.865) (width 0.254) (layer B.Cu) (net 23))
 (segment (start 108.458 57.785) (end 107.188 57.785) (width 0.254) (layer B.Cu) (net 19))
 (segment (start 101.6 63.373) (end 101.6 83.82) (width 0.254) (layer F.Cu) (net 19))
 (segment (start 101.981 62.992) (end 101.6 63.373) (width 0.254) (layer F.Cu) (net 19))
 (via (at 101.981 62.992) (size 0.889) (layers F.Cu B.Cu) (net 19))
 (segment (start 107.188 57.785) (end 101.981 62.992) (width 0.254) (layer B.Cu) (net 19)))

